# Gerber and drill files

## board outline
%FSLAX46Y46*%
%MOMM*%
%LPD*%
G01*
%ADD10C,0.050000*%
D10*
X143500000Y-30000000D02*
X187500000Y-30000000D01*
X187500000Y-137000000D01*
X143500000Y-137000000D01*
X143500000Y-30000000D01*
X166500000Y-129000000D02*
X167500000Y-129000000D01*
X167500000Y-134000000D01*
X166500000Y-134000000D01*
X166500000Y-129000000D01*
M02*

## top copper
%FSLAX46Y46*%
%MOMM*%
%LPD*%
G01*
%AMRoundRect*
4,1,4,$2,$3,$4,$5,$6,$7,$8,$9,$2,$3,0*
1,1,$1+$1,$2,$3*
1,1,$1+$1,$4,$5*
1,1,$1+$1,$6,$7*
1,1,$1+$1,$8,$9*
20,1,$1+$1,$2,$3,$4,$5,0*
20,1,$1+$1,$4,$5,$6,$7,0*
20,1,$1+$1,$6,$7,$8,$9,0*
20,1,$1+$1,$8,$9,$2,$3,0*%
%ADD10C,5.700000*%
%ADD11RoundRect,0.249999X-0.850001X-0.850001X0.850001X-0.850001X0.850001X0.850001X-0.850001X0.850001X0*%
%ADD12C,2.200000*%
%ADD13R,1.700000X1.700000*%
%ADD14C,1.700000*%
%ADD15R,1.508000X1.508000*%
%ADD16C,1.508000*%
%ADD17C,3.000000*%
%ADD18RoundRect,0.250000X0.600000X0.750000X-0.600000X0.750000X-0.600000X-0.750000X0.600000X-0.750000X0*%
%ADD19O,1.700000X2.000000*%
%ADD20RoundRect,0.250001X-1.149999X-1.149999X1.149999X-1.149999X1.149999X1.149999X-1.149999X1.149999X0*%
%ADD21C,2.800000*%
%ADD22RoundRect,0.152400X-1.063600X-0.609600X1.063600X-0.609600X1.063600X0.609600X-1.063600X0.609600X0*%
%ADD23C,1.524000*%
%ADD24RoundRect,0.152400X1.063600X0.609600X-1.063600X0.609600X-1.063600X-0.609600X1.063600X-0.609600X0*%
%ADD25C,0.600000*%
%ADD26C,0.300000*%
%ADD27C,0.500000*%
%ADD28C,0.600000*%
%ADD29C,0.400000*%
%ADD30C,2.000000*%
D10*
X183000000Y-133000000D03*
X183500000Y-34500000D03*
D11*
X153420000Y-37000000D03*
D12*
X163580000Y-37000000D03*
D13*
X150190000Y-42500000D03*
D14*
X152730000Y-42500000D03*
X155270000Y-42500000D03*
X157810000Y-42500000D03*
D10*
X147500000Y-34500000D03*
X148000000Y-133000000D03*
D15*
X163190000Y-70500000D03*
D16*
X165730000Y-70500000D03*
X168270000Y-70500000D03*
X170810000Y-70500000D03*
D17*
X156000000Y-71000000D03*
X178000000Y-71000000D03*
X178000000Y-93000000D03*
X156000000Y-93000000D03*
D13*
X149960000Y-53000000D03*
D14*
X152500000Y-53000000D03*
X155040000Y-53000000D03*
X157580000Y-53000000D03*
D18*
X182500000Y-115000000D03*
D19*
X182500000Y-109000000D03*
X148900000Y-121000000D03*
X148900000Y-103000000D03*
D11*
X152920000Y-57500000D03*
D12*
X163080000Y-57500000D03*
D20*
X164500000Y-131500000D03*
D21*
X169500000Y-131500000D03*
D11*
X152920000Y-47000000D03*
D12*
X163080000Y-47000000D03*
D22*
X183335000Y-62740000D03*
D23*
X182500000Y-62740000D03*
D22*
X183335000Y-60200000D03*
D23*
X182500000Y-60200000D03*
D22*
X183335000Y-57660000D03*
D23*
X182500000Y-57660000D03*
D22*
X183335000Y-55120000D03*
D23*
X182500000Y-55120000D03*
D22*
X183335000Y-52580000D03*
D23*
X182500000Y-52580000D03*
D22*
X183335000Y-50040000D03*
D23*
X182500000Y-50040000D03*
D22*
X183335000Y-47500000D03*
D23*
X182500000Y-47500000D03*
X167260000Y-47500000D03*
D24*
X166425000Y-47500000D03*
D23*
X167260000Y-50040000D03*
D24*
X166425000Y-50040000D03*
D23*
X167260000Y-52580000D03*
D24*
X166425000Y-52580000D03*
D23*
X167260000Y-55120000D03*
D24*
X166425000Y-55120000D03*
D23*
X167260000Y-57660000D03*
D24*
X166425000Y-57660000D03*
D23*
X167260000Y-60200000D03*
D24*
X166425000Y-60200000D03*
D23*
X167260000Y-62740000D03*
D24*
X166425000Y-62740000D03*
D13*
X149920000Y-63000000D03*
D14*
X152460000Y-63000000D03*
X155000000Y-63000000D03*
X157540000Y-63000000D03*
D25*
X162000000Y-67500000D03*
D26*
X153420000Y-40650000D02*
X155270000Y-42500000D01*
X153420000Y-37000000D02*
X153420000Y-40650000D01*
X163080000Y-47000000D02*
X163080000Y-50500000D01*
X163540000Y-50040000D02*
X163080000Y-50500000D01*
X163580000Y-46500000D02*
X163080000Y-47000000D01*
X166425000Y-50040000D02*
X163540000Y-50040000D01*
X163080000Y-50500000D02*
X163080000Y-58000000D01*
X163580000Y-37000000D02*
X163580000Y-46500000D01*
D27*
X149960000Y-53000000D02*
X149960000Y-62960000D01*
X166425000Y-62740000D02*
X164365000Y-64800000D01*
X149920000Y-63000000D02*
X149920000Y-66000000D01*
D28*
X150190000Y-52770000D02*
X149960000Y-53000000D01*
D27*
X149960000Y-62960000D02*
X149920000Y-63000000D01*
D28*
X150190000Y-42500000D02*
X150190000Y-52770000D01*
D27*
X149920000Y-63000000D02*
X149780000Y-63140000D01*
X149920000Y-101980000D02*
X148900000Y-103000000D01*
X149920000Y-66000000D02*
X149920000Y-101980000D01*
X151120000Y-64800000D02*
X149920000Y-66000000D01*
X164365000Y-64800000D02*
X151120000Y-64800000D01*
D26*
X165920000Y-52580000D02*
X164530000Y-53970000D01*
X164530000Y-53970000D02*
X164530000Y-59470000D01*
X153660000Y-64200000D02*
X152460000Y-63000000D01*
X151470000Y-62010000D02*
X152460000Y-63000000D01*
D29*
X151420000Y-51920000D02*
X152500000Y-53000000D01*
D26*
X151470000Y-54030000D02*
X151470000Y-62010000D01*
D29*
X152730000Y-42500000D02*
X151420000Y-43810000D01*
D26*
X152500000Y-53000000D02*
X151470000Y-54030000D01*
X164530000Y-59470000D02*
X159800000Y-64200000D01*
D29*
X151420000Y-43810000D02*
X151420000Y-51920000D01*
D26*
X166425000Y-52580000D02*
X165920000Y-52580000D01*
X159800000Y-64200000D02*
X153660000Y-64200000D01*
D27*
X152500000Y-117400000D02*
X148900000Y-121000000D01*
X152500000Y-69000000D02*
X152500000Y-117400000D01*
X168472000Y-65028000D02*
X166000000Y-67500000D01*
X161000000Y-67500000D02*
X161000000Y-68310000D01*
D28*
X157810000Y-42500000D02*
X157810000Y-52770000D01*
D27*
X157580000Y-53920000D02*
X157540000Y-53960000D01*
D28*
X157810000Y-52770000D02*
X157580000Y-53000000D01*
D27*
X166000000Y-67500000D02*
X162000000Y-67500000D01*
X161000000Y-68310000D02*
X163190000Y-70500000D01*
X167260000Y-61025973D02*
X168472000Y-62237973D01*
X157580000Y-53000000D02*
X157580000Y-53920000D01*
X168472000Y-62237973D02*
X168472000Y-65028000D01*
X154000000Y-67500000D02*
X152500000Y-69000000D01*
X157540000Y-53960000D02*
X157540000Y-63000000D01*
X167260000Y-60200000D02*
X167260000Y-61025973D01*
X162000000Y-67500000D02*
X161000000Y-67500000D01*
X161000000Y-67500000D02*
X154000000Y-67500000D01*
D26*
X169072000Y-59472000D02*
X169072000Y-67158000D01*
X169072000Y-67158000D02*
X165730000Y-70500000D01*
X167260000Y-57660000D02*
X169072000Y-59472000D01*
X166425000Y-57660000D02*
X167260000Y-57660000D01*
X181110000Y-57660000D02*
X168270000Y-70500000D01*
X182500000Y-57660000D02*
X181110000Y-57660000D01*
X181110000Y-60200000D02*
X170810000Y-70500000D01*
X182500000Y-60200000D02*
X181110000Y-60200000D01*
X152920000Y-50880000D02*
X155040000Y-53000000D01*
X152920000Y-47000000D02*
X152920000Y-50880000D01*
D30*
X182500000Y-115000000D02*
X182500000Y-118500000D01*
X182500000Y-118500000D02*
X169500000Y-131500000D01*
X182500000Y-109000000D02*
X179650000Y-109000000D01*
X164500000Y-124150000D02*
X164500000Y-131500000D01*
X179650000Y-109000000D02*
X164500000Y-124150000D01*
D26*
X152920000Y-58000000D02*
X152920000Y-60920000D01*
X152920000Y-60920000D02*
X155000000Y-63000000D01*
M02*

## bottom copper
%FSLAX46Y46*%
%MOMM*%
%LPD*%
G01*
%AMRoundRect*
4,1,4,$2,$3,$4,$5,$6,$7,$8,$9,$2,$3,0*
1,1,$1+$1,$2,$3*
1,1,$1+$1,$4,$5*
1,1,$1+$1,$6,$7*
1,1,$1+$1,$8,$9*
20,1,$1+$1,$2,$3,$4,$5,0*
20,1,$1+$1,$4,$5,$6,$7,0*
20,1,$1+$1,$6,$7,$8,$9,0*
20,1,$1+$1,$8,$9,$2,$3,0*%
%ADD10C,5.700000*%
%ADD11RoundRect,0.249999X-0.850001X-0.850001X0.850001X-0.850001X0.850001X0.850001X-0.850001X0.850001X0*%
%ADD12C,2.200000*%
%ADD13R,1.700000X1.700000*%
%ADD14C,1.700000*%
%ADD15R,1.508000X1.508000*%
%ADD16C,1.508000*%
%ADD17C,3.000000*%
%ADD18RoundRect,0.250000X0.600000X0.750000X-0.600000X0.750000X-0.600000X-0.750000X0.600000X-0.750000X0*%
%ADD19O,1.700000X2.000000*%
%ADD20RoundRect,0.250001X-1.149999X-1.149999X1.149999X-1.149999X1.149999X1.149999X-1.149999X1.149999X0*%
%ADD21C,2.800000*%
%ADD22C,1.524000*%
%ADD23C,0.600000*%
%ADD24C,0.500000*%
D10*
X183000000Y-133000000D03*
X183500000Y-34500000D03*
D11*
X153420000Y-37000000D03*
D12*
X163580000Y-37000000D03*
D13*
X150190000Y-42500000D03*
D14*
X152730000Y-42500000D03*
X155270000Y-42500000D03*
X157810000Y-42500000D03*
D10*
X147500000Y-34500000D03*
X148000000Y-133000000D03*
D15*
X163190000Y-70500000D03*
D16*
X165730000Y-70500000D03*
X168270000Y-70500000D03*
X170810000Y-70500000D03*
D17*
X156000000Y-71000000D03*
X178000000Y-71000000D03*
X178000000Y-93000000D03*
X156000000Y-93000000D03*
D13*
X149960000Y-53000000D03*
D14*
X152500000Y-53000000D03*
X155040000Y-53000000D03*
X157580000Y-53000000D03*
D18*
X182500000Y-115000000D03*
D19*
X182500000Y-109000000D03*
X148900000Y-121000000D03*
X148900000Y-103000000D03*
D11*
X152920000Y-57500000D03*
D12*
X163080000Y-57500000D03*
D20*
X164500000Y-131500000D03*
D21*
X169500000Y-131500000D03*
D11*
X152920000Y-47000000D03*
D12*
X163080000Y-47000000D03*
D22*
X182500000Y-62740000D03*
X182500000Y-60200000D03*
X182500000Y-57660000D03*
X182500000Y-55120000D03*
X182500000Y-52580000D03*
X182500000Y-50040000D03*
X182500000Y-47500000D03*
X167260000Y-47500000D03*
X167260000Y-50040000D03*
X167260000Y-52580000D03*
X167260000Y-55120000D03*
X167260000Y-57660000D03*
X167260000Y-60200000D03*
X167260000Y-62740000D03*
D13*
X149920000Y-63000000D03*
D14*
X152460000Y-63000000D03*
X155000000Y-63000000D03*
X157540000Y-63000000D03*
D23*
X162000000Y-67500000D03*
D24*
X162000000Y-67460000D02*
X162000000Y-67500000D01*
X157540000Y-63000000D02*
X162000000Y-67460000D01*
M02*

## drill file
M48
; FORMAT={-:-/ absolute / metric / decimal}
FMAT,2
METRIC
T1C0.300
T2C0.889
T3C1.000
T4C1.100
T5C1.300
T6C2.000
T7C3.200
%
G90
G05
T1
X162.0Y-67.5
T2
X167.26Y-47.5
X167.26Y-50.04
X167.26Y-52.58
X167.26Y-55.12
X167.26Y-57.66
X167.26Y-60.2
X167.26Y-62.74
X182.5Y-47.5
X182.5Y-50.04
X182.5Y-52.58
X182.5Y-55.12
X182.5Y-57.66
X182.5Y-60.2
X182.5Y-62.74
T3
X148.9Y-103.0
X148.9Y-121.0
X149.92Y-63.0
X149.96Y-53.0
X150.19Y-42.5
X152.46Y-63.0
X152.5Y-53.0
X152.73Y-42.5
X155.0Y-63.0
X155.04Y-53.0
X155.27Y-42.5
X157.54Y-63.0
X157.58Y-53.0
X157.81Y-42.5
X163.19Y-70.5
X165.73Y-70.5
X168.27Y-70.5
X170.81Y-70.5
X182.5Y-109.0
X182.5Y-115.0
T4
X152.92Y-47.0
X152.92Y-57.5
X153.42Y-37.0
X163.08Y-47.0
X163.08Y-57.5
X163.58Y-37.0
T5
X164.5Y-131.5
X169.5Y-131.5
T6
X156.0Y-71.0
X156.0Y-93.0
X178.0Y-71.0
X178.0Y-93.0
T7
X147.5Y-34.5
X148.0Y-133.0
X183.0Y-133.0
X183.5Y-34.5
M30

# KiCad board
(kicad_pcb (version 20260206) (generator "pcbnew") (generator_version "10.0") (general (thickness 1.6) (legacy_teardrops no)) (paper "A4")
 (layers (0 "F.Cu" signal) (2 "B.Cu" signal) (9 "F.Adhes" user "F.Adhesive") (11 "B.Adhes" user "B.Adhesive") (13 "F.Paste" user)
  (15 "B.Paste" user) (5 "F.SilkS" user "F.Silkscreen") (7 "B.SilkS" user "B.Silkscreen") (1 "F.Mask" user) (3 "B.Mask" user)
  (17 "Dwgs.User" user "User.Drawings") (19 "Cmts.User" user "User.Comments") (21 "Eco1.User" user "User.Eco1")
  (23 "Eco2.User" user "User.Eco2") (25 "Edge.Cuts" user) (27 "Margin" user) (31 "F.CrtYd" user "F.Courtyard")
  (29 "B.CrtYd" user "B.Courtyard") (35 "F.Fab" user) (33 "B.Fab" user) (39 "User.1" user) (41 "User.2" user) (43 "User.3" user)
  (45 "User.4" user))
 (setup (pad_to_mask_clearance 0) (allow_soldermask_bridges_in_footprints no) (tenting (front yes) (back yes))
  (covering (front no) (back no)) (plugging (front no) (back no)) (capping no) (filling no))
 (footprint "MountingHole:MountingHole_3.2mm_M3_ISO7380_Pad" (layer "F.Cu") (at 183 133)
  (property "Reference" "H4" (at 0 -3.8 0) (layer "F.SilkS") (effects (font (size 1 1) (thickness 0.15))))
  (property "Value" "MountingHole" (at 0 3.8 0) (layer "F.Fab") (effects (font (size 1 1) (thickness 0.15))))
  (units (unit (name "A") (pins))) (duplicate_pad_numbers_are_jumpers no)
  (pad "1" thru_hole circle (at 0 0) (size 5.7 5.7) (drill 3.2) (layers "*.Cu" "*.Mask") (remove_unused_layers no) (zone_connect 2)))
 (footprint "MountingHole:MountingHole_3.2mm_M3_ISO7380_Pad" (layer "F.Cu") (at 183.5 34.5)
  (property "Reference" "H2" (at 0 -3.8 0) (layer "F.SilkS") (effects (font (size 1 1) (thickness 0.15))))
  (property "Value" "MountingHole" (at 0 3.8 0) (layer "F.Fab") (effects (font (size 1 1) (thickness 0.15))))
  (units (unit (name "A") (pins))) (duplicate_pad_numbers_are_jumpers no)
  (pad "1" thru_hole circle (at 0 0) (size 5.7 5.7) (drill 3.2) (layers "*.Cu" "*.Mask") (remove_unused_layers no) (zone_connect 2)))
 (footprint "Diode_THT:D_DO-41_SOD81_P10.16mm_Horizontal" (layer "F.Cu") (at 153.42 37)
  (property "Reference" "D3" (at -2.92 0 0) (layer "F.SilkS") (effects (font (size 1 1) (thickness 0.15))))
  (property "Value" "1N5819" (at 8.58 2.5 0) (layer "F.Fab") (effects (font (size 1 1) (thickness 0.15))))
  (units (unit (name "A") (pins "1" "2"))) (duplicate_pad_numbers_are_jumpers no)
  (pad "1" thru_hole roundrect (at 0 0) (size 2.2 2.2) (drill 1.1) (layers "*.Cu" "*.Mask") (remove_unused_layers no)
   (roundrect_rratio 0.113636) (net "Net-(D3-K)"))
  (pad "2" thru_hole circle (at 10.16 0) (size 2.2 2.2) (drill 1.1) (layers "*.Cu" "*.Mask") (remove_unused_layers no) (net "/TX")))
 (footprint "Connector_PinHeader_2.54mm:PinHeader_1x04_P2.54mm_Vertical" (layer "F.Cu") (at 150.19 42.5 90)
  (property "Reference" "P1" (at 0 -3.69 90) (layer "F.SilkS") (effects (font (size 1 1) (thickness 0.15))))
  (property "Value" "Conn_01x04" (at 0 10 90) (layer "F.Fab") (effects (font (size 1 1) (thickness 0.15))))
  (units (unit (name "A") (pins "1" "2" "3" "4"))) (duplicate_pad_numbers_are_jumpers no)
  (pad "1" thru_hole rect (at 0 0 90) (size 1.7 1.7) (drill 1) (layers "*.Cu" "*.Mask") (remove_unused_layers no) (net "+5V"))
  (pad "2" thru_hole circle (at 0 2.54 90) (size 1.7 1.7) (drill 1) (layers "*.Cu" "*.Mask") (remove_unused_layers no) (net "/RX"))
  (pad "3" thru_hole circle (at 0 5.08 90) (size 1.7 1.7) (drill 1) (layers "*.Cu" "*.Mask") (remove_unused_layers no) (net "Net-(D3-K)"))
  (pad "4" thru_hole circle (at 0 7.62 90) (size 1.7 1.7) (drill 1) (layers "*.Cu" "*.Mask") (remove_unused_layers no) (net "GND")))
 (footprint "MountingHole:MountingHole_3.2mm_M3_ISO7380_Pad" (layer "F.Cu") (at 147.5 34.5)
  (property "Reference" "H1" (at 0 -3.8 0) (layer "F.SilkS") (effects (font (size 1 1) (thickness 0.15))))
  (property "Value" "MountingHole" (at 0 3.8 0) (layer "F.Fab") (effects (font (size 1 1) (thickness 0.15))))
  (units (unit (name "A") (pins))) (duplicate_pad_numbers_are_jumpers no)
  (pad "1" thru_hole circle (at 0 0) (size 5.7 5.7) (drill 3.2) (layers "*.Cu" "*.Mask") (remove_unused_layers no) (zone_connect 2)))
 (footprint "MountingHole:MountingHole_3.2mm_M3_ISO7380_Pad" (layer "F.Cu") (at 148 133)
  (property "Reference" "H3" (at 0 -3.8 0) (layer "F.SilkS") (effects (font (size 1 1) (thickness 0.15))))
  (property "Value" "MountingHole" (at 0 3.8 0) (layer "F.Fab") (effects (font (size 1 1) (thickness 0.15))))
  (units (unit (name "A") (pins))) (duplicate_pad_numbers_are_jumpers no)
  (pad "1" thru_hole circle (at 0 0) (size 5.7 5.7) (drill 3.2) (layers "*.Cu" "*.Mask") (remove_unused_layers no) (zone_connect 2)))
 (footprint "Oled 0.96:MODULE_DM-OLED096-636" (layer "F.Cu") (at 167 82)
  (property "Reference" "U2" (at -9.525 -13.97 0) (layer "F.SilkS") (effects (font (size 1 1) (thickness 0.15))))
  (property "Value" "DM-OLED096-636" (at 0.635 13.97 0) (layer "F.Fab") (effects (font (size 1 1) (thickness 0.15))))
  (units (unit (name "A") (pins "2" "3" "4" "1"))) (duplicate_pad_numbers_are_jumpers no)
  (pad "1" thru_hole rect (at -3.81 -11.5) (size 1.508 1.508) (drill 1) (layers "*.Cu" "*.Mask") (remove_unused_layers no) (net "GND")
   (solder_mask_margin 0.102))
  (pad "2" thru_hole circle (at -1.27 -11.5) (size 1.508 1.508) (drill 1) (layers "*.Cu" "*.Mask") (remove_unused_layers no) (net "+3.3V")
   (solder_mask_margin 0.102))
  (pad "3" thru_hole circle (at 1.27 -11.5) (size 1.508 1.508) (drill 1) (layers "*.Cu" "*.Mask") (remove_unused_layers no) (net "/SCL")
   (solder_mask_margin 0.102))
  (pad "4" thru_hole circle (at 3.81 -11.5) (size 1.508 1.508) (drill 1) (layers "*.Cu" "*.Mask") (remove_unused_layers no) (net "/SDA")
   (solder_mask_margin 0.102))
  (pad "S1" thru_hole circle (at -11 -11) (size 3 3) (drill 2) (layers "*.Cu" "*.Mask") (remove_unused_layers no) (solder_mask_margin 0.102))
  (pad "S2" thru_hole circle (at 11 -11) (size 3 3) (drill 2) (layers "*.Cu" "*.Mask") (remove_unused_layers no) (solder_mask_margin 0.102))
  (pad "S3" thru_hole circle (at 11 11) (size 3 3) (drill 2) (layers "*.Cu" "*.Mask") (remove_unused_layers no) (solder_mask_margin 0.102))
  (pad "S4" thru_hole circle (at -11 11) (size 3 3) (drill 2) (layers "*.Cu" "*.Mask") (remove_unused_layers no) (solder_mask_margin 0.102)))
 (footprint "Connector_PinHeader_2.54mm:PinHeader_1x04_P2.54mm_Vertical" (layer "F.Cu") (at 149.96 53 90)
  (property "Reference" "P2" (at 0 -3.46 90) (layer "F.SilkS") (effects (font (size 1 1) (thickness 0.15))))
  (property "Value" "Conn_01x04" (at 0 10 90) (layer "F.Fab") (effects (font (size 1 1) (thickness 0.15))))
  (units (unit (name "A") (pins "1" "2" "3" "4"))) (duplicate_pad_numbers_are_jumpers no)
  (pad "1" thru_hole rect (at 0 0 90) (size 1.7 1.7) (drill 1) (layers "*.Cu" "*.Mask") (remove_unused_layers no) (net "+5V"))
  (pad "2" thru_hole circle (at 0 2.54 90) (size 1.7 1.7) (drill 1) (layers "*.Cu" "*.Mask") (remove_unused_layers no) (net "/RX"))
  (pad "3" thru_hole circle (at 0 5.08 90) (size 1.7 1.7) (drill 1) (layers "*.Cu" "*.Mask") (remove_unused_layers no) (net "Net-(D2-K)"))
  (pad "4" thru_hole circle (at 0 7.62 90) (size 1.7 1.7) (drill 1) (layers "*.Cu" "*.Mask") (remove_unused_layers no) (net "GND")))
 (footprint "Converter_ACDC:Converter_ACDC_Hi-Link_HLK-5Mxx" (layer "F.Cu") (at 182.5 115 180)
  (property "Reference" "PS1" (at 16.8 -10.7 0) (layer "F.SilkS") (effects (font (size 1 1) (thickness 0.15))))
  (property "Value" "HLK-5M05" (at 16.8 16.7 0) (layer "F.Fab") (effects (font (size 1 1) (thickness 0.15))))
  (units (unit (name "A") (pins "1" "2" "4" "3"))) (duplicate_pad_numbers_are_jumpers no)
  (pad "1" thru_hole roundrect (at 0 0 180) (size 1.7 2) (drill 1) (layers "*.Cu" "*.Mask") (remove_unused_layers no)
   (roundrect_rratio 0.147059) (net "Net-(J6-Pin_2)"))
  (pad "2" thru_hole oval (at 0 6 180) (size 1.7 2) (drill 1) (layers "*.Cu" "*.Mask") (remove_unused_layers no) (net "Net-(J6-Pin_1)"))
  (pad "3" thru_hole oval (at 33.6 -6 180) (size 1.7 2) (drill 1) (layers "*.Cu" "*.Mask") (remove_unused_layers no) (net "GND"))
  (pad "4" thru_hole oval (at 33.6 12 180) (size 1.7 2) (drill 1) (layers "*.Cu" "*.Mask") (remove_unused_layers no) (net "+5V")))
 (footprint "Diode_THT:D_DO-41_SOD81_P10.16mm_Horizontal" (layer "F.Cu") (at 152.92 57.5)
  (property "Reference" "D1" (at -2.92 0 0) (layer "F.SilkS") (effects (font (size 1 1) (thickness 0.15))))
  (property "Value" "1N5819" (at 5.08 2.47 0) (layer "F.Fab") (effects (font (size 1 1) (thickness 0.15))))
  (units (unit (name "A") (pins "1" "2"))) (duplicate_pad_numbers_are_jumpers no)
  (pad "1" thru_hole roundrect (at 0 0) (size 2.2 2.2) (drill 1.1) (layers "*.Cu" "*.Mask") (remove_unused_layers no)
   (roundrect_rratio 0.113636) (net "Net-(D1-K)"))
  (pad "2" thru_hole circle (at 10.16 0) (size 2.2 2.2) (drill 1.1) (layers "*.Cu" "*.Mask") (remove_unused_layers no) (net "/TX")))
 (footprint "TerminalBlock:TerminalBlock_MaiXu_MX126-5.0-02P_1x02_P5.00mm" (layer "F.Cu") (at 164.5 131.5)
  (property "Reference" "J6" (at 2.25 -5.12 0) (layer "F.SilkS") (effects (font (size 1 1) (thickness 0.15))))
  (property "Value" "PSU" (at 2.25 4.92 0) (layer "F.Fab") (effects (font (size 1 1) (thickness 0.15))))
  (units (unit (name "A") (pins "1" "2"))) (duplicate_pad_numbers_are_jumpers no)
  (pad "1" thru_hole roundrect (at 0 0) (size 2.8 2.8) (drill 1.3) (layers "*.Cu" "*.Mask") (remove_unused_layers no)
   (roundrect_rratio 0.089286) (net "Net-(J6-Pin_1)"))
  (pad "2" thru_hole circle (at 5 0) (size 2.8 2.8) (drill 1.3) (layers "*.Cu" "*.Mask") (remove_unused_layers no) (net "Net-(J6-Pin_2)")))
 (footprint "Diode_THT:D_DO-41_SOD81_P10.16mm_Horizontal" (layer "F.Cu") (at 152.92 47)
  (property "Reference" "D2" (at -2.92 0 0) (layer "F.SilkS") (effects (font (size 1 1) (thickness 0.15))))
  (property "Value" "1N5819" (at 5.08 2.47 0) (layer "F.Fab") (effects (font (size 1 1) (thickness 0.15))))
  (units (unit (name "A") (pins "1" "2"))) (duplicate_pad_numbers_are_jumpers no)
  (pad "1" thru_hole roundrect (at 0 0) (size 2.2 2.2) (drill 1.1) (layers "*.Cu" "*.Mask") (remove_unused_layers no)
   (roundrect_rratio 0.113636) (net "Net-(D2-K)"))
  (pad "2" thru_hole circle (at 10.16 0) (size 2.2 2.2) (drill 1.1) (layers "*.Cu" "*.Mask") (remove_unused_layers no) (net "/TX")))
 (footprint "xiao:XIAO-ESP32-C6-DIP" (layer "F.Cu") (at 174.88 55.12 -90)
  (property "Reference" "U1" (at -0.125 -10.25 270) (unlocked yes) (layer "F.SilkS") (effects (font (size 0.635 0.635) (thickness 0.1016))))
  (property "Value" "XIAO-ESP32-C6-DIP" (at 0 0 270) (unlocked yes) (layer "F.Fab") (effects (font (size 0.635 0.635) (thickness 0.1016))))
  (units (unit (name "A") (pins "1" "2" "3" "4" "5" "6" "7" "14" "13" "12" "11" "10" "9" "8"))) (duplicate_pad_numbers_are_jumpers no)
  (pad "1" smd roundrect (at 7.62 -8.455) (size 2.432 1.524) (layers "F.Cu" "F.Mask") (roundrect_rratio 0.1)
   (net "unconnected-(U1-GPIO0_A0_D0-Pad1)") (thermal_bridge_angle 45))
  (pad "1" thru_hole circle (at 7.62 -7.62) (size 1.524 1.524) (drill 0.889) (layers "*.Cu" "*.Mask") (remove_unused_layers no)
   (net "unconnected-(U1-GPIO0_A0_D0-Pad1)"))
  (pad "2" smd roundrect (at 5.08 -8.455) (size 2.432 1.524) (layers "F.Cu" "F.Mask") (roundrect_rratio 0.1) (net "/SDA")
   (thermal_bridge_angle 45))
  (pad "2" thru_hole circle (at 5.08 -7.62) (size 1.524 1.524) (drill 0.889) (layers "*.Cu" "*.Mask") (remove_unused_layers no) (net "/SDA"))
  (pad "3" smd roundrect (at 2.54 -8.455) (size 2.432 1.524) (layers "F.Cu" "F.Mask") (roundrect_rratio 0.1) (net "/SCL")
   (thermal_bridge_angle 45))
  (pad "3" thru_hole circle (at 2.54 -7.62) (size 1.524 1.524) (drill 0.889) (layers "*.Cu" "*.Mask") (remove_unused_layers no) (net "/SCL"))
  (pad "4" smd roundrect (at 0 -8.455) (size 2.432 1.524) (layers "F.Cu" "F.Mask") (roundrect_rratio 0.1)
   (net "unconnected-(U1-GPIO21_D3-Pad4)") (thermal_bridge_angle 45))
  (pad "4" thru_hole circle (at 0 -7.62) (size 1.524 1.524) (drill 0.889) (layers "*.Cu" "*.Mask") (remove_unused_layers no)
   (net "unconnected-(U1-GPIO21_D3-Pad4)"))
  (pad "5" smd roundrect (at -2.54 -8.455) (size 2.432 1.524) (layers "F.Cu" "F.Mask") (roundrect_rratio 0.1)
   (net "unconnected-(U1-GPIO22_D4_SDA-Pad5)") (thermal_bridge_angle 45))
  (pad "5" thru_hole circle (at -2.54 -7.62) (size 1.524 1.524) (drill 0.889) (layers "*.Cu" "*.Mask") (remove_unused_layers no)
   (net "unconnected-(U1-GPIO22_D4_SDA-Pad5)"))
  (pad "6" smd roundrect (at -5.08 -8.455) (size 2.432 1.524) (layers "F.Cu" "F.Mask") (roundrect_rratio 0.1)
   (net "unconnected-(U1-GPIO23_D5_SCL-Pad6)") (thermal_bridge_angle 45))
  (pad "6" thru_hole circle (at -5.08 -7.62) (size 1.524 1.524) (drill 0.889) (layers "*.Cu" "*.Mask") (remove_unused_layers no)
   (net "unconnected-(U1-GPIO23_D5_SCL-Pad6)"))
  (pad "7" smd roundrect (at -7.62 -8.455) (size 2.432 1.524) (layers "F.Cu" "F.Mask") (roundrect_rratio 0.1)
   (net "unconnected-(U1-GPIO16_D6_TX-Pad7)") (thermal_bridge_angle 45))
  (pad "7" thru_hole circle (at -7.62 -7.62) (size 1.524 1.524) (drill 0.889) (layers "*.Cu" "*.Mask") (remove_unused_layers no)
   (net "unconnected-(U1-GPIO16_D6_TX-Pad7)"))
  (pad "8" thru_hole circle (at -7.62 7.62 180) (size 1.524 1.524) (drill 0.889) (layers "*.Cu" "*.Mask") (remove_unused_layers no)
   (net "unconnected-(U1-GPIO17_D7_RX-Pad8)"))
  (pad "8" smd roundrect (at -7.62 8.455 180) (size 2.432 1.524) (layers "F.Cu" "F.Mask") (roundrect_rratio 0.1)
   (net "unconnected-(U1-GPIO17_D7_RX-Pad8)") (thermal_bridge_angle 45))
  (pad "9" thru_hole circle (at -5.08 7.62 180) (size 1.524 1.524) (drill 0.889) (layers "*.Cu" "*.Mask") (remove_unused_layers no)
   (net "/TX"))
  (pad "9" smd roundrect (at -5.08 8.455 180) (size 2.432 1.524) (layers "F.Cu" "F.Mask") (roundrect_rratio 0.1) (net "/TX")
   (thermal_bridge_angle 45))
  (pad "10" thru_hole circle (at -2.54 7.62 180) (size 1.524 1.524) (drill 0.889) (layers "*.Cu" "*.Mask") (remove_unused_layers no)
   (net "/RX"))
  (pad "10" smd roundrect (at -2.54 8.455 180) (size 2.432 1.524) (layers "F.Cu" "F.Mask") (roundrect_rratio 0.1) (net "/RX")
   (thermal_bridge_angle 45))
  (pad "11" thru_hole circle (at 0 7.62 180) (size 1.524 1.524) (drill 0.889) (layers "*.Cu" "*.Mask") (remove_unused_layers no)
   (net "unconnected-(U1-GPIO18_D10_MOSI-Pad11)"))
  (pad "11" smd roundrect (at 0 8.455 180) (size 2.432 1.524) (layers "F.Cu" "F.Mask") (roundrect_rratio 0.1)
   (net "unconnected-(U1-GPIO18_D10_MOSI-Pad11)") (thermal_bridge_angle 45))
  (pad "12" thru_hole circle (at 2.54 7.62 180) (size 1.524 1.524) (drill 0.889) (layers "*.Cu" "*.Mask") (remove_unused_layers no)
   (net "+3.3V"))
  (pad "12" smd roundrect (at 2.54 8.455 180) (size 2.432 1.524) (layers "F.Cu" "F.Mask") (roundrect_rratio 0.1) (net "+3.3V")
   (thermal_bridge_angle 45))
  (pad "13" thru_hole circle (at 5.08 7.62 180) (size 1.524 1.524) (drill 0.889) (layers "*.Cu" "*.Mask") (remove_unused_layers no)
   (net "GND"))
  (pad "13" smd roundrect (at 5.08 8.455 180) (size 2.432 1.524) (layers "F.Cu" "F.Mask") (roundrect_rratio 0.1) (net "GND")
   (thermal_bridge_angle 45))
  (pad "14" thru_hole circle (at 7.62 7.62 180) (size 1.524 1.524) (drill 0.889) (layers "*.Cu" "*.Mask") (remove_unused_layers no)
   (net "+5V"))
  (pad "14" smd roundrect (at 7.62 8.455 180) (size 2.432 1.524) (layers "F.Cu" "F.Mask") (roundrect_rratio 0.1) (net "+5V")
   (thermal_bridge_angle 45)))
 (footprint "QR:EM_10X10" (layer "F.Cu") (at 173.75 36.5)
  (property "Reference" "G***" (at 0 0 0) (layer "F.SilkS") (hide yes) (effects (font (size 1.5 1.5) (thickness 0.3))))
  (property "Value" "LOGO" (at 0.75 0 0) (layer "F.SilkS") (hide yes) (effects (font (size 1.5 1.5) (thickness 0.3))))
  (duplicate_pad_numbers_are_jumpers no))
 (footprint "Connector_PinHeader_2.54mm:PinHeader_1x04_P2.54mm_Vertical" (layer "F.Cu") (at 149.92 63 90)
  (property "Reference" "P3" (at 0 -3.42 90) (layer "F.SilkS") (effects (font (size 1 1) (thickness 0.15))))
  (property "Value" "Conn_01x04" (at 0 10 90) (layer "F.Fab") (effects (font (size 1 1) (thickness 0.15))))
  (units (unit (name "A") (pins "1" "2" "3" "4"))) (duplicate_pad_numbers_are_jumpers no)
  (pad "1" thru_hole rect (at 0 0 90) (size 1.7 1.7) (drill 1) (layers "*.Cu" "*.Mask") (remove_unused_layers no) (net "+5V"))
  (pad "2" thru_hole circle (at 0 2.54 90) (size 1.7 1.7) (drill 1) (layers "*.Cu" "*.Mask") (remove_unused_layers no) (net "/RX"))
  (pad "3" thru_hole circle (at 0 5.08 90) (size 1.7 1.7) (drill 1) (layers "*.Cu" "*.Mask") (remove_unused_layers no) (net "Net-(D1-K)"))
  (pad "4" thru_hole circle (at 0 7.62 90) (size 1.7 1.7) (drill 1) (layers "*.Cu" "*.Mask") (remove_unused_layers no) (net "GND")))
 (gr_rect (start 143.5 30) (end 187.5 137) (stroke (width 0.05) (type default)) (fill no) (layer "Edge.Cuts"))
 (gr_rect (start 166.5 129) (end 167.5 134) (stroke (width 0.05) (type default)) (fill no) (layer "Edge.Cuts"))
 (segment (start 153.42 40.65) (end 155.27 42.5) (width 0.3) (layer "F.Cu") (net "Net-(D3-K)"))
 (segment (start 153.42 37) (end 153.42 40.65) (width 0.3) (layer "F.Cu") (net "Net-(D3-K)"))
 (segment (start 163.08 47) (end 163.08 50.5) (width 0.3) (layer "F.Cu") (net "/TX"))
 (segment (start 163.54 50.04) (end 163.08 50.5) (width 0.3) (layer "F.Cu") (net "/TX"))
 (segment (start 163.58 46.5) (end 163.08 47) (width 0.3) (layer "F.Cu") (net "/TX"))
 (segment (start 166.425 50.04) (end 163.54 50.04) (width 0.3) (layer "F.Cu") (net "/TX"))
 (segment (start 163.08 50.5) (end 163.08 58) (width 0.3) (layer "F.Cu") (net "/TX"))
 (segment (start 163.58 37) (end 163.58 46.5) (width 0.3) (layer "F.Cu") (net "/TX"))
 (segment (start 149.96 53) (end 149.96 62.96) (width 0.5) (layer "F.Cu") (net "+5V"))
 (segment (start 166.425 62.74) (end 164.365 64.8) (width 0.5) (layer "F.Cu") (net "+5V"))
 (segment (start 149.92 63) (end 149.92 66) (width 0.5) (layer "F.Cu") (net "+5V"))
 (segment (start 150.19 52.77) (end 149.96 53) (width 0.6) (layer "F.Cu") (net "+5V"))
 (segment (start 149.96 62.96) (end 149.92 63) (width 0.5) (layer "F.Cu") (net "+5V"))
 (segment (start 150.19 42.5) (end 150.19 52.77) (width 0.6) (layer "F.Cu") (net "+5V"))
 (segment (start 149.92 63) (end 149.78 63.14) (width 0.5) (layer "F.Cu") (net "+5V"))
 (segment (start 149.92 101.98) (end 148.9 103) (width 0.5) (layer "F.Cu") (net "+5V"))
 (segment (start 149.92 66) (end 149.92 101.98) (width 0.5) (layer "F.Cu") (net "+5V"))
 (segment (start 151.12 64.8) (end 149.92 66) (width 0.5) (layer "F.Cu") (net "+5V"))
 (segment (start 164.365 64.8) (end 151.12 64.8) (width 0.5) (layer "F.Cu") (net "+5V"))
 (segment (start 165.92 52.58) (end 164.53 53.97) (width 0.3) (layer "F.Cu") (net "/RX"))
 (segment (start 164.53 53.97) (end 164.53 59.47) (width 0.3) (layer "F.Cu") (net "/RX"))
 (segment (start 153.66 64.2) (end 152.46 63) (width 0.3) (layer "F.Cu") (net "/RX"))
 (segment (start 151.47 62.01) (end 152.46 63) (width 0.3) (layer "F.Cu") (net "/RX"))
 (segment (start 151.42 51.92) (end 152.5 53) (width 0.4) (layer "F.Cu") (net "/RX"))
 (segment (start 151.47 54.03) (end 151.47 62.01) (width 0.3) (layer "F.Cu") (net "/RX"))
 (segment (start 152.73 42.5) (end 151.42 43.81) (width 0.4) (layer "F.Cu") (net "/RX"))
 (segment (start 152.5 53) (end 151.47 54.03) (width 0.3) (layer "F.Cu") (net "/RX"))
 (segment (start 164.53 59.47) (end 159.8 64.2) (width 0.3) (layer "F.Cu") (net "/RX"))
 (segment (start 151.42 43.81) (end 151.42 51.92) (width 0.4) (layer "F.Cu") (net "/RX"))
 (segment (start 166.425 52.58) (end 165.92 52.58) (width 0.3) (layer "F.Cu") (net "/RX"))
 (segment (start 159.8 64.2) (end 153.66 64.2) (width 0.3) (layer "F.Cu") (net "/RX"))
 (segment (start 152.5 117.4) (end 148.9 121) (width 0.5) (layer "F.Cu") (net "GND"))
 (segment (start 152.5 69) (end 152.5 117.4) (width 0.5) (layer "F.Cu") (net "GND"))
 (segment (start 168.472 65.028) (end 166 67.5) (width 0.5) (layer "F.Cu") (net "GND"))
 (segment (start 161 67.5) (end 161 68.31) (width 0.5) (layer "F.Cu") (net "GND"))
 (segment (start 157.81 42.5) (end 157.81 52.77) (width 0.6) (layer "F.Cu") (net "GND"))
 (segment (start 157.58 53.92) (end 157.54 53.96) (width 0.5) (layer "F.Cu") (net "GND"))
 (segment (start 157.81 52.77) (end 157.58 53) (width 0.6) (layer "F.Cu") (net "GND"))
 (segment (start 166 67.5) (end 162 67.5) (width 0.5) (layer "F.Cu") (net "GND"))
 (segment (start 161 68.31) (end 163.19 70.5) (width 0.5) (layer "F.Cu") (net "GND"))
 (segment (start 167.26 61.025973) (end 168.472 62.237973) (width 0.5) (layer "F.Cu") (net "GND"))
 (segment (start 157.58 53) (end 157.58 53.92) (width 0.5) (layer "F.Cu") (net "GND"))
 (segment (start 168.472 62.237973) (end 168.472 65.028) (width 0.5) (layer "F.Cu") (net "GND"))
 (segment (start 154 67.5) (end 152.5 69) (width 0.5) (layer "F.Cu") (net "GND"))
 (segment (start 157.54 53.96) (end 157.54 63) (width 0.5) (layer "F.Cu") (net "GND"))
 (segment (start 167.26 60.2) (end 167.26 61.025973) (width 0.5) (layer "F.Cu") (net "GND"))
 (segment (start 162 67.5) (end 161 67.5) (width 0.5) (layer "F.Cu") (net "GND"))
 (segment (start 161 67.5) (end 154 67.5) (width 0.5) (layer "F.Cu") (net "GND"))
 (via (at 162 67.5) (size 0.6) (drill 0.3) (layers "F.Cu" "B.Cu") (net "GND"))
 (segment (start 162 67.46) (end 162 67.5) (width 0.5) (layer "B.Cu") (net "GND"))
 (segment (start 157.54 63) (end 162 67.46) (width 0.5) (layer "B.Cu") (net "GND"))
 (segment (start 169.072 59.472) (end 169.072 67.158) (width 0.3) (layer "F.Cu") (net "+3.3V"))
 (segment (start 169.072 67.158) (end 165.73 70.5) (width 0.3) (layer "F.Cu") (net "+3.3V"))
 (segment (start 167.26 57.66) (end 169.072 59.472) (width 0.3) (layer "F.Cu") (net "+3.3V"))
 (segment (start 166.425 57.66) (end 167.26 57.66) (width 0.3) (layer "F.Cu") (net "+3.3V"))
 (segment (start 181.11 57.66) (end 168.27 70.5) (width 0.3) (layer "F.Cu") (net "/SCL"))
 (segment (start 182.5 57.66) (end 181.11 57.66) (width 0.3) (layer "F.Cu") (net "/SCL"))
 (segment (start 181.11 60.2) (end 170.81 70.5) (width 0.3) (layer "F.Cu") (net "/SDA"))
 (segment (start 182.5 60.2) (end 181.11 60.2) (width 0.3) (layer "F.Cu") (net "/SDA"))
 (segment (start 152.92 50.88) (end 155.04 53) (width 0.3) (layer "F.Cu") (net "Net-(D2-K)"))
 (segment (start 152.92 47) (end 152.92 50.88) (width 0.3) (layer "F.Cu") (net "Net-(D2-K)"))
 (segment (start 182.5 115) (end 182.5 118.5) (width 2) (layer "F.Cu") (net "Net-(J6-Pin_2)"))
 (segment (start 182.5 118.5) (end 169.5 131.5) (width 2) (layer "F.Cu") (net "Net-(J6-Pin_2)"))
 (segment (start 182.5 109) (end 179.65 109) (width 2) (layer "F.Cu") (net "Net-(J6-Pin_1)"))
 (segment (start 164.5 124.15) (end 164.5 131.5) (width 2) (layer "F.Cu") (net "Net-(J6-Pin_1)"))
 (segment (start 179.65 109) (end 164.5 124.15) (width 2) (layer "F.Cu") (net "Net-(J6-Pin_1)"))
 (segment (start 152.92 58) (end 152.92 60.92) (width 0.3) (layer "F.Cu") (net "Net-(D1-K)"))
 (segment (start 152.92 60.92) (end 155 63) (width 0.3) (layer "F.Cu") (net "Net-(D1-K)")))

